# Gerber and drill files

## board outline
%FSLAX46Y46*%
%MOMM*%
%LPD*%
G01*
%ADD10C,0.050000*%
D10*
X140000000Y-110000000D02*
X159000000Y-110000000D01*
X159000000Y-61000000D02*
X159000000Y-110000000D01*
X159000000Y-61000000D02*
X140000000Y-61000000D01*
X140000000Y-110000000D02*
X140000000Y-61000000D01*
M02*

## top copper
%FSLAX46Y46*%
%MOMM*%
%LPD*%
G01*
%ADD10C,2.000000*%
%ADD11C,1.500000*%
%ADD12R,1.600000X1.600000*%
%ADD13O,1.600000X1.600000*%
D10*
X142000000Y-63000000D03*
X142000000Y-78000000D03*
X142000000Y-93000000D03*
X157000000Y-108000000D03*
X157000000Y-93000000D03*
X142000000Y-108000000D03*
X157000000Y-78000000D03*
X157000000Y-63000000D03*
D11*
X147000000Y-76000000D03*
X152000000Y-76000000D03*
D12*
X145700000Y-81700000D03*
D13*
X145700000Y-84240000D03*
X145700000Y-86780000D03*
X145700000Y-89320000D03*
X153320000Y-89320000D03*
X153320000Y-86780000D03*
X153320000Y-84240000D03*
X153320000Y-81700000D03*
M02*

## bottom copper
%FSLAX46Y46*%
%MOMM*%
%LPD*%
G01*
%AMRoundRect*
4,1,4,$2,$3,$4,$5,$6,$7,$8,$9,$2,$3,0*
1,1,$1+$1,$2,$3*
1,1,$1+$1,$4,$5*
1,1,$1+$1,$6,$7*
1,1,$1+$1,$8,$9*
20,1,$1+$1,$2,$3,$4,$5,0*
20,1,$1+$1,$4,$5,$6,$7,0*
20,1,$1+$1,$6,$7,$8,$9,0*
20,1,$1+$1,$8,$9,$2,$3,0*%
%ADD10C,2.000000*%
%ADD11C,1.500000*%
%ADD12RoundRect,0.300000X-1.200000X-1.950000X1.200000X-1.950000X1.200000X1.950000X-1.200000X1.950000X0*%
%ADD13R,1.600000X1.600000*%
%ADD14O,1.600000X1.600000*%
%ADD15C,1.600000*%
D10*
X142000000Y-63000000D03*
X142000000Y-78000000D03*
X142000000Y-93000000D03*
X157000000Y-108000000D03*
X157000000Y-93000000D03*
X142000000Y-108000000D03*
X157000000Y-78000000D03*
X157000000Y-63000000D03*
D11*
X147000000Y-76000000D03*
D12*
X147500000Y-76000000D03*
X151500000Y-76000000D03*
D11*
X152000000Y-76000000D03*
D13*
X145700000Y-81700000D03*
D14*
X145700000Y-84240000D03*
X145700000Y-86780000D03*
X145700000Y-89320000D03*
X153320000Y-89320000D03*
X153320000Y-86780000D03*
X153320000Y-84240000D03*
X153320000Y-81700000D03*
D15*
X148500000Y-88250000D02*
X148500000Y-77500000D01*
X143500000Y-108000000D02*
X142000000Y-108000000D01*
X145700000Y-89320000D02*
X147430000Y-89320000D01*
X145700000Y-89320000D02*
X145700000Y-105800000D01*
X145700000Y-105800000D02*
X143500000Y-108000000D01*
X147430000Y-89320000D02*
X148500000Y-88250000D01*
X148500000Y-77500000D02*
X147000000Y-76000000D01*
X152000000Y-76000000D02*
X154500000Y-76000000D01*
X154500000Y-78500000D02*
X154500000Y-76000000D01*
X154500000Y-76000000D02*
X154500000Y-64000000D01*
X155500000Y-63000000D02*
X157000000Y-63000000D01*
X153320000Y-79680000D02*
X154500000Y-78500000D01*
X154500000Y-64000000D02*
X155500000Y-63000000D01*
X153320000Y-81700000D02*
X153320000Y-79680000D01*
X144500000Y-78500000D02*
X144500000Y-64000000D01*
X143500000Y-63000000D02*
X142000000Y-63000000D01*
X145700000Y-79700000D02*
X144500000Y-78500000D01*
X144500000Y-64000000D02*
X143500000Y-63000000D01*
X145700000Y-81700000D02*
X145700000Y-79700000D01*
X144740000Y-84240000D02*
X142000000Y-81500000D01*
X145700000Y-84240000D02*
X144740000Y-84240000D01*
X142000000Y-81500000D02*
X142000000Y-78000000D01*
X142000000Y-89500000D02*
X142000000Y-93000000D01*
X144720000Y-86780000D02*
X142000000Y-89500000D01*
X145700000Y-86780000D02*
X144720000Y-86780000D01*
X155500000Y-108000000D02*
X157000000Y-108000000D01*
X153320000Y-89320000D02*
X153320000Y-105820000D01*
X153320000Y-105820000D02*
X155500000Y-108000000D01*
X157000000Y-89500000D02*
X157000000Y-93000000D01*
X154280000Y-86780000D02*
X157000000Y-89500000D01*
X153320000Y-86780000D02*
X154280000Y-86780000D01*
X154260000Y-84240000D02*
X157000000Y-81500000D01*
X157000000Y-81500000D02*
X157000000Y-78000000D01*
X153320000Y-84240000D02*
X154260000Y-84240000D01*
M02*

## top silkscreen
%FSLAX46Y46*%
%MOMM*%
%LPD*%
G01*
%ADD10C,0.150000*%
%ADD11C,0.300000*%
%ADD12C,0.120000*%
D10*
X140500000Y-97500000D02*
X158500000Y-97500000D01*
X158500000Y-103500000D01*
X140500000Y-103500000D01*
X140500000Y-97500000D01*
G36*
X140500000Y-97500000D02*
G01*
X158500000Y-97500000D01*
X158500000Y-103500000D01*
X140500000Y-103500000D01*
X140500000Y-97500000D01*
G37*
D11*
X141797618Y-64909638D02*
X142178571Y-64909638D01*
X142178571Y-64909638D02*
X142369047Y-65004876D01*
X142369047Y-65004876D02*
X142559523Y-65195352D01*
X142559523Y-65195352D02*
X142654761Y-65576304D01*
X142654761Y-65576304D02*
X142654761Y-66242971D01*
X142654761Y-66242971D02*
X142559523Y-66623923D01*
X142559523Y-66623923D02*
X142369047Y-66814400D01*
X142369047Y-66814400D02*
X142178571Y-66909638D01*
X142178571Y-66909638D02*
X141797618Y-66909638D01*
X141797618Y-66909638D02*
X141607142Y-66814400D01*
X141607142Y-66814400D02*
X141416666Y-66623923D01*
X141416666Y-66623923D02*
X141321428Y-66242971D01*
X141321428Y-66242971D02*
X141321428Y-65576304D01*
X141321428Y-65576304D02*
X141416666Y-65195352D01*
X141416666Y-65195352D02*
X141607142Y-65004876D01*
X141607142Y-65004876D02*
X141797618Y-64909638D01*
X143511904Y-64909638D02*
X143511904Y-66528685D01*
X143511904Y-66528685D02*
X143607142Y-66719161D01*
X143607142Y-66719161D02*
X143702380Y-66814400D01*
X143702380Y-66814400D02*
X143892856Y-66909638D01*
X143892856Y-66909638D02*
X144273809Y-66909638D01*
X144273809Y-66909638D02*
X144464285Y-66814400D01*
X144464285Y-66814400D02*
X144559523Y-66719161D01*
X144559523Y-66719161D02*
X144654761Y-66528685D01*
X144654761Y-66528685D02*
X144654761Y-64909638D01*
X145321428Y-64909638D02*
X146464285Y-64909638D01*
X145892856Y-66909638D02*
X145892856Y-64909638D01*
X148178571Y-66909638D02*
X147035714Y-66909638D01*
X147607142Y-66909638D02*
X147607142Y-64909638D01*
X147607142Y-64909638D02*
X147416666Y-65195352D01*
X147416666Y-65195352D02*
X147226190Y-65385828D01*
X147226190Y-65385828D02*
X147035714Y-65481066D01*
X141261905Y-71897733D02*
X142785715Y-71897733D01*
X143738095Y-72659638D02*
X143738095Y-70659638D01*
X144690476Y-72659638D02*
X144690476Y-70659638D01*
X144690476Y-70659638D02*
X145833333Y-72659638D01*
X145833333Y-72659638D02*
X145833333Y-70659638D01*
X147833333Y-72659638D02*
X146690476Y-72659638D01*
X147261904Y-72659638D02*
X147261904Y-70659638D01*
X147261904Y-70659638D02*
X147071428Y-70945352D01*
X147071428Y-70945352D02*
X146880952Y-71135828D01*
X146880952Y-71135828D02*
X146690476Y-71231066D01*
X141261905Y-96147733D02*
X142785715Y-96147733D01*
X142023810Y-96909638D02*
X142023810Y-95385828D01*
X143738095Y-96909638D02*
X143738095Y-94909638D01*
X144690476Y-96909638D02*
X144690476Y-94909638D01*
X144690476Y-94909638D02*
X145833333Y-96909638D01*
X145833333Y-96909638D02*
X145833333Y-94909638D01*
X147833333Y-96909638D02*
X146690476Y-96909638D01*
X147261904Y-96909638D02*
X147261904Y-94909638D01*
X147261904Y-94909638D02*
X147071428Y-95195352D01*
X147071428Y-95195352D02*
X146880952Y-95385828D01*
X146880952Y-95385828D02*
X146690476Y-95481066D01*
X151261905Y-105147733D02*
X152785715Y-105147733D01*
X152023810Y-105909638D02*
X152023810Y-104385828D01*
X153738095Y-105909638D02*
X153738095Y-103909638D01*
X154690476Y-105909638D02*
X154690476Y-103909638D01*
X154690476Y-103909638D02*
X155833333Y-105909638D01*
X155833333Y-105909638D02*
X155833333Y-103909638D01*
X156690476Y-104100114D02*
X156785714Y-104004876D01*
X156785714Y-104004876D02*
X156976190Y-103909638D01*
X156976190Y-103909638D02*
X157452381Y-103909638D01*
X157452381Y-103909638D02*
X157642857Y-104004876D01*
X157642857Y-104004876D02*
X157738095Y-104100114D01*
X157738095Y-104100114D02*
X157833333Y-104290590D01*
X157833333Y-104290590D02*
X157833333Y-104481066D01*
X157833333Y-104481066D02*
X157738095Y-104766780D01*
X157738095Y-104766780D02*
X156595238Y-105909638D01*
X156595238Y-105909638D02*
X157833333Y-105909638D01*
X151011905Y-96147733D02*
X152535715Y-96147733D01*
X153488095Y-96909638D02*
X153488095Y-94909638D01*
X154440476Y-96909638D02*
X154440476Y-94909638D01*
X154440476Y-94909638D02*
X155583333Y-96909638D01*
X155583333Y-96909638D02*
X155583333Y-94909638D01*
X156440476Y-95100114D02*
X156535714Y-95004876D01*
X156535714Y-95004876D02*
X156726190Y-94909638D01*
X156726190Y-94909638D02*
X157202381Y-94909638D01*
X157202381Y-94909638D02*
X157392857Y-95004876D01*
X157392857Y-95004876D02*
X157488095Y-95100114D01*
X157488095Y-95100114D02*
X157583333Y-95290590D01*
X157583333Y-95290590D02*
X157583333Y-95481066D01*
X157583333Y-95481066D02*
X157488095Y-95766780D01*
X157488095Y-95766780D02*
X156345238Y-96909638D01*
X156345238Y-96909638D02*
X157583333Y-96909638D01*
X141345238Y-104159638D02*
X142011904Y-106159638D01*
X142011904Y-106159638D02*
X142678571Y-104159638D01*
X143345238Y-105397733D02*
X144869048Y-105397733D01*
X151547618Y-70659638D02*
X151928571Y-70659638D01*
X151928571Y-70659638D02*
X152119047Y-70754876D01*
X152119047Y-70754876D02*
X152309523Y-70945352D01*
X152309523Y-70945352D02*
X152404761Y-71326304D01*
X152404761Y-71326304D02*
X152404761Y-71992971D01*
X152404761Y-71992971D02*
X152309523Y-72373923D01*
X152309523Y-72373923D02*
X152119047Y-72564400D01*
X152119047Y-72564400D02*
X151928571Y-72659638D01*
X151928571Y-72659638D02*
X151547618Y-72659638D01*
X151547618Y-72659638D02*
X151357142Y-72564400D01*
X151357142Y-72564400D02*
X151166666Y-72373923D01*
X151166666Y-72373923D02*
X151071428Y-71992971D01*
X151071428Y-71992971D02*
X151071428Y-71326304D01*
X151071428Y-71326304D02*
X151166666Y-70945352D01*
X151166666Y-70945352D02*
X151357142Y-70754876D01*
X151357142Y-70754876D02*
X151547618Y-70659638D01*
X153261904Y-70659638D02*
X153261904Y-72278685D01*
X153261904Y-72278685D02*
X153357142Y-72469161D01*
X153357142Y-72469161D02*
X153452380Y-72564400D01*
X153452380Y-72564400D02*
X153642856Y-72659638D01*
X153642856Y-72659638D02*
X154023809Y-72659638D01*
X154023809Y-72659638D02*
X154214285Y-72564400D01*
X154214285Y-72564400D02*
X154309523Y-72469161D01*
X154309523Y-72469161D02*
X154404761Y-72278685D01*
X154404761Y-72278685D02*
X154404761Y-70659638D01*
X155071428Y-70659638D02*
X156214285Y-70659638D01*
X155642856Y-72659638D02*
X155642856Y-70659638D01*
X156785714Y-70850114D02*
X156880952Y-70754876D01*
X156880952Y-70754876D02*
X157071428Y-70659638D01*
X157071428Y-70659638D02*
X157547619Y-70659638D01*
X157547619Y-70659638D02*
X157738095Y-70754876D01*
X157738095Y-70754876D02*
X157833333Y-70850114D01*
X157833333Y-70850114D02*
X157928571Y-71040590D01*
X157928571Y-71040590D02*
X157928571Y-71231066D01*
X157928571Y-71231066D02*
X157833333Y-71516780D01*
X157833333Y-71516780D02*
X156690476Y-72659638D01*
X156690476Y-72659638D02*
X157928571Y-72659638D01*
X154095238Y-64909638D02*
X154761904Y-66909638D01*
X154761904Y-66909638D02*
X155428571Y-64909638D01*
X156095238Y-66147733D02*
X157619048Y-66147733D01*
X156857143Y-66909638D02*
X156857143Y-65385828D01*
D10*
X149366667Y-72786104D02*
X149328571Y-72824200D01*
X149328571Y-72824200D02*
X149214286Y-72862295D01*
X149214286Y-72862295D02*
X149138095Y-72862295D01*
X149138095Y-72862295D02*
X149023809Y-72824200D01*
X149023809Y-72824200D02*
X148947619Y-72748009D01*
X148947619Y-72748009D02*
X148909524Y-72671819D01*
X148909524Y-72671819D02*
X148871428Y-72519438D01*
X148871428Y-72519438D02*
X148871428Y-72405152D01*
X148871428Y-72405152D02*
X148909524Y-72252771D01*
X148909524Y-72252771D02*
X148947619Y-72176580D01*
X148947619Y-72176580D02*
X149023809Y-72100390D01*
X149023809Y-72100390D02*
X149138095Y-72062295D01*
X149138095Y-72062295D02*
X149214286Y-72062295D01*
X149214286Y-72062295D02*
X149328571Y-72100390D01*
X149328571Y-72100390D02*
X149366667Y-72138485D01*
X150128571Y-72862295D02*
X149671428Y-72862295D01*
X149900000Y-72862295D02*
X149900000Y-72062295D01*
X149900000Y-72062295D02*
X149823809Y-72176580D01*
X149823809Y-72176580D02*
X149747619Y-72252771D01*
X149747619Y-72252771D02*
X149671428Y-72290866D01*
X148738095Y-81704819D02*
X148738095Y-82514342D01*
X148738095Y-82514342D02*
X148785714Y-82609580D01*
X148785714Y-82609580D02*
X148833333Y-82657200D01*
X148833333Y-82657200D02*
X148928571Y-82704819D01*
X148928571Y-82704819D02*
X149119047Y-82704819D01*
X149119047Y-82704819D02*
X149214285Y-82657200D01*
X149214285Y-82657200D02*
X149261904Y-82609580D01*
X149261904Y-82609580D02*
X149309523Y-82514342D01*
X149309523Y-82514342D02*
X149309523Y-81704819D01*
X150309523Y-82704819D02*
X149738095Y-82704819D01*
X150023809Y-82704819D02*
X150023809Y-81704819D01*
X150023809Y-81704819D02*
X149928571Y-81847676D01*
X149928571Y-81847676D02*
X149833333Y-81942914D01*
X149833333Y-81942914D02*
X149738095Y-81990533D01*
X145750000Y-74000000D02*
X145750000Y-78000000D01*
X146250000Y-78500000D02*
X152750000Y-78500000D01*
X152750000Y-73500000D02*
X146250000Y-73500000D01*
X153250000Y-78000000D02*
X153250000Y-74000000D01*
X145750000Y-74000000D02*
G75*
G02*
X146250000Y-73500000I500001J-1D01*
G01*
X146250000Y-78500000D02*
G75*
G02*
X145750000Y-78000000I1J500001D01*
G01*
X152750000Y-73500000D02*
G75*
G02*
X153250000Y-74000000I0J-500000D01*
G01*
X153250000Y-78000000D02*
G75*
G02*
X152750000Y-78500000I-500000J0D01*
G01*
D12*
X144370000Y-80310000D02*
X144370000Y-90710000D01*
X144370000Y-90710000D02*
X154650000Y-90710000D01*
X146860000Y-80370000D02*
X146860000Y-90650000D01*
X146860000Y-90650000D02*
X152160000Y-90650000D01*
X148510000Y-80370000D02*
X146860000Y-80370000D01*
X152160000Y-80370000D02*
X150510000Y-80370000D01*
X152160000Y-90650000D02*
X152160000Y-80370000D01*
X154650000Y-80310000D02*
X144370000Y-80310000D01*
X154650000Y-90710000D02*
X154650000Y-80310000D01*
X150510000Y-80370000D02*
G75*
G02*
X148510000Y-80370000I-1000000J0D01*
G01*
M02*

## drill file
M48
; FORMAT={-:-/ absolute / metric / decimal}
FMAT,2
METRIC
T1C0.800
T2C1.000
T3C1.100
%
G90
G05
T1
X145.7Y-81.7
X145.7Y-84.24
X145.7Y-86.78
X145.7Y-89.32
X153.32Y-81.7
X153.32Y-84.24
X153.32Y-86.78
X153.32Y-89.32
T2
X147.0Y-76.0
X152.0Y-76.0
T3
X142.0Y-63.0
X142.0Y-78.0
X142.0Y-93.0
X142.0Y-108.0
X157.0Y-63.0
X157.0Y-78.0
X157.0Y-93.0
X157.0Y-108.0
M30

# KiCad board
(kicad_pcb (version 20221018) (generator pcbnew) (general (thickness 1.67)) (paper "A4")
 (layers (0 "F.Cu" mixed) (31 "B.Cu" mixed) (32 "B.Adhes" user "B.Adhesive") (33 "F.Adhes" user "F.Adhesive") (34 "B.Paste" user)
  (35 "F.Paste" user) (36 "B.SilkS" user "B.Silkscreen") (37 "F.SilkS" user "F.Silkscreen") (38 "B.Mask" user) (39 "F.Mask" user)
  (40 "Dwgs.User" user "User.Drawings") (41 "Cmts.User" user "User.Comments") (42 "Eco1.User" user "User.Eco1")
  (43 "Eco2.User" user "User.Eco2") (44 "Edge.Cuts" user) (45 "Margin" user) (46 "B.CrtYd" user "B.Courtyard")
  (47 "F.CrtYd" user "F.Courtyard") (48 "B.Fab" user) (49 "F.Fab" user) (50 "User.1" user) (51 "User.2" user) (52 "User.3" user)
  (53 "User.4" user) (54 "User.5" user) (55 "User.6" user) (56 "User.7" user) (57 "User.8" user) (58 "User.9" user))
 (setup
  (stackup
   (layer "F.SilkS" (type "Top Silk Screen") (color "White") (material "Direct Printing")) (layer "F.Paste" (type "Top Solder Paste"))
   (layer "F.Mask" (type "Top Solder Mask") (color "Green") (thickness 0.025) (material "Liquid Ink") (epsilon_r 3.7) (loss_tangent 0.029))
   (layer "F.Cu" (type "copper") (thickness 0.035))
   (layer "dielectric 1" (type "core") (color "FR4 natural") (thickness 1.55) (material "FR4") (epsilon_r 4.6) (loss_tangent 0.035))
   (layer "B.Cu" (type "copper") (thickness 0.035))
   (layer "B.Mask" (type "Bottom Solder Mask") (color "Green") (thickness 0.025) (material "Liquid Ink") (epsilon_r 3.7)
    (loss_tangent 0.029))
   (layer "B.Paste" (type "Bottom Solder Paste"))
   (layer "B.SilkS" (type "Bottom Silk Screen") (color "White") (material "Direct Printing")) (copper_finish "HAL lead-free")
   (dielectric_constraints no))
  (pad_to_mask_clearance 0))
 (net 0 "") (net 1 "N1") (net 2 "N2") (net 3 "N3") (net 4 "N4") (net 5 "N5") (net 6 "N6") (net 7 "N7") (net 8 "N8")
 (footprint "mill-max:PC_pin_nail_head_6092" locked (layer "F.Cu") (at 142 63)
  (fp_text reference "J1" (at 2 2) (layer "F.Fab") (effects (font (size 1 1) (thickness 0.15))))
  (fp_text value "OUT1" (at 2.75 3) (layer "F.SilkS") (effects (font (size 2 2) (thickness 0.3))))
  (pad "1" thru_hole circle locked (at 0 0) (size 2 2) (drill 1.1) (layers "*.Cu" "*.Mask") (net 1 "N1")))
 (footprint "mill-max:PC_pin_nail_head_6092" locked (layer "F.Cu") (at 142 78)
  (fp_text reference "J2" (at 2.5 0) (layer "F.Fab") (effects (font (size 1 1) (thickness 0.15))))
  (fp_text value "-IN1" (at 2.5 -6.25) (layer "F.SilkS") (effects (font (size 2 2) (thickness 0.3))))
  (pad "1" thru_hole circle locked (at 0 0) (size 2 2) (drill 1.1) (layers "*.Cu" "*.Mask") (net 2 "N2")))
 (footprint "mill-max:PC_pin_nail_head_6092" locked (layer "F.Cu") (at 142 93)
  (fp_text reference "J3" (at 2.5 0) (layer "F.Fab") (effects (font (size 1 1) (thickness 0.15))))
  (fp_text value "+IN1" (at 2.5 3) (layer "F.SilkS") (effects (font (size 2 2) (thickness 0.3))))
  (pad "1" thru_hole circle locked (at 0 0) (size 2 2) (drill 1.1) (layers "*.Cu" "*.Mask") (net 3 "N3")))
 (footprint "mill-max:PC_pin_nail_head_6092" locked (layer "F.Cu") (at 157 108)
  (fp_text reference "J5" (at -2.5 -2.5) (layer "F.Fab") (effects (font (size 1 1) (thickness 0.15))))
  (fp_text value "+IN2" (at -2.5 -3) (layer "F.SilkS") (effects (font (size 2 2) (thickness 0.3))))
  (pad "1" thru_hole circle locked (at 0 0) (size 2 2) (drill 1.1) (layers "*.Cu" "*.Mask") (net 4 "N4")))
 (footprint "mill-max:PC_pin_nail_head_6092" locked (layer "F.Cu") (at 157 93)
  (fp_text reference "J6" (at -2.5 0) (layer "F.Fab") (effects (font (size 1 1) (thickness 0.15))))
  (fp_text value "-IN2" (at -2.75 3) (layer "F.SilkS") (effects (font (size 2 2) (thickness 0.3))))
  (pad "1" thru_hole circle locked (at 0 0) (size 2 2) (drill 1.1) (layers "*.Cu" "*.Mask") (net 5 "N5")))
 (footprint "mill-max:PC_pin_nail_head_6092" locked (layer "F.Cu") (at 142 108)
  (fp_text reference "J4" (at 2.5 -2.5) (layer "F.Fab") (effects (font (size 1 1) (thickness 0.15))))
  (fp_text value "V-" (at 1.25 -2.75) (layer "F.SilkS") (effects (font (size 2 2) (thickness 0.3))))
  (pad "1" thru_hole circle locked (at 0 0) (size 2 2) (drill 1.1) (layers "*.Cu" "*.Mask") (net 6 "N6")))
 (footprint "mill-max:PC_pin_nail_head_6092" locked (layer "F.Cu") (at 157 78)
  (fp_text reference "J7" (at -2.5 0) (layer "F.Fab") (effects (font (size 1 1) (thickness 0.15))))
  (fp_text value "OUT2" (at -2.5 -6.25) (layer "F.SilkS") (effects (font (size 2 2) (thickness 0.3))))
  (pad "1" thru_hole circle locked (at 0 0) (size 2 2) (drill 1.1) (layers "*.Cu" "*.Mask") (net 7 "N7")))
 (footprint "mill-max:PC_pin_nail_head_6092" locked (layer "F.Cu") (at 157 63)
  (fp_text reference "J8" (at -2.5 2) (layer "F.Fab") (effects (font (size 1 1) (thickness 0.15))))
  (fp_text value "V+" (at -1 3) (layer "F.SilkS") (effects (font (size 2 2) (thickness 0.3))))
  (pad "1" thru_hole circle locked (at 0 0) (size 2 2) (drill 1.1) (layers "*.Cu" "*.Mask") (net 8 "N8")))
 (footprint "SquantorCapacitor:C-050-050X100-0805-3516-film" (layer "F.Cu") (at 149.5 76)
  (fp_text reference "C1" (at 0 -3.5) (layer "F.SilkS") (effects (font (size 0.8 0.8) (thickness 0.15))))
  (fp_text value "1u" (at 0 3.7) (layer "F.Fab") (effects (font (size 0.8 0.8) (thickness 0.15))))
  (fp_line (start -3.75 -2) (end -3.75 2) (stroke (width 0.15) (type solid)) (layer "F.SilkS"))
  (fp_line (start -3.25 2.5) (end 3.25 2.5) (stroke (width 0.15) (type solid)) (layer "F.SilkS"))
  (fp_line (start 3.25 -2.5) (end -3.25 -2.5) (stroke (width 0.15) (type solid)) (layer "F.SilkS"))
  (fp_line (start 3.75 2) (end 3.75 -2) (stroke (width 0.15) (type solid)) (layer "F.SilkS"))
  (fp_arc (start -3.75 -2) (mid -3.603553 -2.353553) (end -3.25 -2.5) (stroke (width 0.15) (type solid)) (layer "F.SilkS"))
  (fp_arc (start -3.25 2.5) (mid -3.603553 2.353553) (end -3.75 2) (stroke (width 0.15) (type solid)) (layer "F.SilkS"))
  (fp_arc (start 3.25 -2.5) (mid 3.603553 -2.353553) (end 3.75 -2) (stroke (width 0.15) (type solid)) (layer "F.SilkS"))
  (fp_arc (start 3.75 2) (mid 3.603553 2.353553) (end 3.25 2.5) (stroke (width 0.15) (type solid)) (layer "F.SilkS"))
  (pad "1" thru_hole circle (at -2.5 0) (size 1.5 1.5) (drill 1) (layers "*.Cu" "*.Mask") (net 6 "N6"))
  (pad "1" smd roundrect (at -2 0) (size 3 4.5) (layers "B.Cu" "B.Paste" "B.Mask") (roundrect_rratio 0.1) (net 6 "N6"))
  (pad "2" smd roundrect (at 2 0) (size 3 4.5) (layers "B.Cu" "B.Paste" "B.Mask") (roundrect_rratio 0.1) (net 8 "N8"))
  (pad "2" thru_hole circle (at 2.5 0) (size 1.5 1.5) (drill 1) (layers "*.Cu" "*.Mask") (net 8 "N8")))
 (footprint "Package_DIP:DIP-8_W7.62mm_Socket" (layer "F.Cu") (at 145.7 81.7)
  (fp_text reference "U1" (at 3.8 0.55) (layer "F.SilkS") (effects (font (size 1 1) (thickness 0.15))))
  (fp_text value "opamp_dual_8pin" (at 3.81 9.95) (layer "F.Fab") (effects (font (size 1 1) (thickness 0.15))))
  (fp_line (start -1.33 -1.39) (end -1.33 9.01) (stroke (width 0.12) (type solid)) (layer "F.SilkS"))
  (fp_line (start -1.33 9.01) (end 8.95 9.01) (stroke (width 0.12) (type solid)) (layer "F.SilkS"))
  (fp_line (start 1.16 -1.33) (end 1.16 8.95) (stroke (width 0.12) (type solid)) (layer "F.SilkS"))
  (fp_line (start 1.16 8.95) (end 6.46 8.95) (stroke (width 0.12) (type solid)) (layer "F.SilkS"))
  (fp_line (start 2.81 -1.33) (end 1.16 -1.33) (stroke (width 0.12) (type solid)) (layer "F.SilkS"))
  (fp_line (start 6.46 -1.33) (end 4.81 -1.33) (stroke (width 0.12) (type solid)) (layer "F.SilkS"))
  (fp_line (start 6.46 8.95) (end 6.46 -1.33) (stroke (width 0.12) (type solid)) (layer "F.SilkS"))
  (fp_line (start 8.95 -1.39) (end -1.33 -1.39) (stroke (width 0.12) (type solid)) (layer "F.SilkS"))
  (fp_line (start 8.95 9.01) (end 8.95 -1.39) (stroke (width 0.12) (type solid)) (layer "F.SilkS"))
  (fp_arc (start 4.81 -1.33) (mid 3.81 -0.33) (end 2.81 -1.33) (stroke (width 0.12) (type solid)) (layer "F.SilkS"))
  (pad "1" thru_hole rect (at 0 0) (size 1.6 1.6) (drill 0.8) (layers "*.Cu" "*.Mask") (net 1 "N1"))
  (pad "2" thru_hole oval (at 0 2.54) (size 1.6 1.6) (drill 0.8) (layers "*.Cu" "*.Mask") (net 2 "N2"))
  (pad "3" thru_hole oval (at 0 5.08) (size 1.6 1.6) (drill 0.8) (layers "*.Cu" "*.Mask") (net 3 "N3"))
  (pad "4" thru_hole oval (at 0 7.62) (size 1.6 1.6) (drill 0.8) (layers "*.Cu" "*.Mask") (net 6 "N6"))
  (pad "5" thru_hole oval (at 7.62 7.62) (size 1.6 1.6) (drill 0.8) (layers "*.Cu" "*.Mask") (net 4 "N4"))
  (pad "6" thru_hole oval (at 7.62 5.08) (size 1.6 1.6) (drill 0.8) (layers "*.Cu" "*.Mask") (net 5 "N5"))
  (pad "7" thru_hole oval (at 7.62 2.54) (size 1.6 1.6) (drill 0.8) (layers "*.Cu" "*.Mask") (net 7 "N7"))
  (pad "8" thru_hole oval (at 7.62 0) (size 1.6 1.6) (drill 0.8) (layers "*.Cu" "*.Mask") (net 8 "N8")))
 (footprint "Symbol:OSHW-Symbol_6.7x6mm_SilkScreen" (layer "B.Cu") (at 149 105 180)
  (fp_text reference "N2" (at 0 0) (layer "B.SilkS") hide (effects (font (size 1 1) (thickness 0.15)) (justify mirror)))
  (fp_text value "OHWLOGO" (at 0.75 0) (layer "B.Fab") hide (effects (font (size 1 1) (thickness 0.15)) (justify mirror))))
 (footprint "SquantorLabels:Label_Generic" (layer "B.Cu") (at 148 109)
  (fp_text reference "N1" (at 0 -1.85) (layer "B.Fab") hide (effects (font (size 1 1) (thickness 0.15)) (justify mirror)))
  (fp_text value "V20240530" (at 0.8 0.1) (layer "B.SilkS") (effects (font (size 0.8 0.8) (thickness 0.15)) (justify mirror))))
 (gr_rect (start 140.5 97.5) (end 158.5 103.5) (stroke (width 0.15) (type solid)) (fill solid) (layer "F.SilkS"))
 (gr_line (start 140 110) (end 159 110) (stroke (width 0.05) (type solid)) (layer "Edge.Cuts"))
 (gr_line (start 159 61) (end 159 110) (stroke (width 0.05) (type solid)) (layer "Edge.Cuts"))
 (gr_line (start 159 61) (end 140 61) (stroke (width 0.05) (type solid)) (layer "Edge.Cuts"))
 (gr_line (start 140 110) (end 140 61) (stroke (width 0.05) (type solid)) (layer "Edge.Cuts"))
 (segment (start 148.5 88.25) (end 148.5 77.5) (width 1.6) (layer "B.Cu") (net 6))
 (segment (start 143.5 108) (end 142 108) (width 1.6) (layer "B.Cu") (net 6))
 (segment (start 145.7 89.32) (end 147.43 89.32) (width 1.6) (layer "B.Cu") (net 6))
 (segment (start 145.7 89.32) (end 145.7 105.8) (width 1.6) (layer "B.Cu") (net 6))
 (segment (start 145.7 105.8) (end 143.5 108) (width 1.6) (layer "B.Cu") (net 6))
 (segment (start 147.43 89.32) (end 148.5 88.25) (width 1.6) (layer "B.Cu") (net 6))
 (segment (start 148.5 77.5) (end 147 76) (width 1.6) (layer "B.Cu") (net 6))
 (segment (start 152 76) (end 154.5 76) (width 1.6) (layer "B.Cu") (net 8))
 (segment (start 154.5 78.5) (end 154.5 76) (width 1.6) (layer "B.Cu") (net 8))
 (segment (start 154.5 76) (end 154.5 64) (width 1.6) (layer "B.Cu") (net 8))
 (segment (start 155.5 63) (end 157 63) (width 1.6) (layer "B.Cu") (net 8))
 (segment (start 153.32 79.68) (end 154.5 78.5) (width 1.6) (layer "B.Cu") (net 8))
 (segment (start 154.5 64) (end 155.5 63) (width 1.6) (layer "B.Cu") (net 8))
 (segment (start 153.32 81.7) (end 153.32 79.68) (width 1.6) (layer "B.Cu") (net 8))
 (segment (start 144.5 78.5) (end 144.5 64) (width 1.6) (layer "B.Cu") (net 1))
 (segment (start 143.5 63) (end 142 63) (width 1.6) (layer "B.Cu") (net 1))
 (segment (start 145.7 79.7) (end 144.5 78.5) (width 1.6) (layer "B.Cu") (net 1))
 (segment (start 144.5 64) (end 143.5 63) (width 1.6) (layer "B.Cu") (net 1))
 (segment (start 145.7 81.7) (end 145.7 79.7) (width 1.6) (layer "B.Cu") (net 1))
 (segment (start 144.74 84.24) (end 142 81.5) (width 1.6) (layer "B.Cu") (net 2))
 (segment (start 145.7 84.24) (end 144.74 84.24) (width 1.6) (layer "B.Cu") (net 2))
 (segment (start 142 81.5) (end 142 78) (width 1.6) (layer "B.Cu") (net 2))
 (segment (start 142 89.5) (end 142 93) (width 1.6) (layer "B.Cu") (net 3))
 (segment (start 144.72 86.78) (end 142 89.5) (width 1.6) (layer "B.Cu") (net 3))
 (segment (start 145.7 86.78) (end 144.72 86.78) (width 1.6) (layer "B.Cu") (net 3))
 (segment (start 155.5 108) (end 157 108) (width 1.6) (layer "B.Cu") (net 4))
 (segment (start 153.32 89.32) (end 153.32 105.82) (width 1.6) (layer "B.Cu") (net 4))
 (segment (start 153.32 105.82) (end 155.5 108) (width 1.6) (layer "B.Cu") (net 4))
 (segment (start 157 89.5) (end 157 93) (width 1.6) (layer "B.Cu") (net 5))
 (segment (start 154.28 86.78) (end 157 89.5) (width 1.6) (layer "B.Cu") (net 5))
 (segment (start 153.32 86.78) (end 154.28 86.78) (width 1.6) (layer "B.Cu") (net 5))
 (segment (start 154.26 84.24) (end 157 81.5) (width 1.6) (layer "B.Cu") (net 7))
 (segment (start 157 81.5) (end 157 78) (width 1.6) (layer "B.Cu") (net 7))
 (segment (start 153.32 84.24) (end 154.26 84.24) (width 1.6) (layer "B.Cu") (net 7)))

